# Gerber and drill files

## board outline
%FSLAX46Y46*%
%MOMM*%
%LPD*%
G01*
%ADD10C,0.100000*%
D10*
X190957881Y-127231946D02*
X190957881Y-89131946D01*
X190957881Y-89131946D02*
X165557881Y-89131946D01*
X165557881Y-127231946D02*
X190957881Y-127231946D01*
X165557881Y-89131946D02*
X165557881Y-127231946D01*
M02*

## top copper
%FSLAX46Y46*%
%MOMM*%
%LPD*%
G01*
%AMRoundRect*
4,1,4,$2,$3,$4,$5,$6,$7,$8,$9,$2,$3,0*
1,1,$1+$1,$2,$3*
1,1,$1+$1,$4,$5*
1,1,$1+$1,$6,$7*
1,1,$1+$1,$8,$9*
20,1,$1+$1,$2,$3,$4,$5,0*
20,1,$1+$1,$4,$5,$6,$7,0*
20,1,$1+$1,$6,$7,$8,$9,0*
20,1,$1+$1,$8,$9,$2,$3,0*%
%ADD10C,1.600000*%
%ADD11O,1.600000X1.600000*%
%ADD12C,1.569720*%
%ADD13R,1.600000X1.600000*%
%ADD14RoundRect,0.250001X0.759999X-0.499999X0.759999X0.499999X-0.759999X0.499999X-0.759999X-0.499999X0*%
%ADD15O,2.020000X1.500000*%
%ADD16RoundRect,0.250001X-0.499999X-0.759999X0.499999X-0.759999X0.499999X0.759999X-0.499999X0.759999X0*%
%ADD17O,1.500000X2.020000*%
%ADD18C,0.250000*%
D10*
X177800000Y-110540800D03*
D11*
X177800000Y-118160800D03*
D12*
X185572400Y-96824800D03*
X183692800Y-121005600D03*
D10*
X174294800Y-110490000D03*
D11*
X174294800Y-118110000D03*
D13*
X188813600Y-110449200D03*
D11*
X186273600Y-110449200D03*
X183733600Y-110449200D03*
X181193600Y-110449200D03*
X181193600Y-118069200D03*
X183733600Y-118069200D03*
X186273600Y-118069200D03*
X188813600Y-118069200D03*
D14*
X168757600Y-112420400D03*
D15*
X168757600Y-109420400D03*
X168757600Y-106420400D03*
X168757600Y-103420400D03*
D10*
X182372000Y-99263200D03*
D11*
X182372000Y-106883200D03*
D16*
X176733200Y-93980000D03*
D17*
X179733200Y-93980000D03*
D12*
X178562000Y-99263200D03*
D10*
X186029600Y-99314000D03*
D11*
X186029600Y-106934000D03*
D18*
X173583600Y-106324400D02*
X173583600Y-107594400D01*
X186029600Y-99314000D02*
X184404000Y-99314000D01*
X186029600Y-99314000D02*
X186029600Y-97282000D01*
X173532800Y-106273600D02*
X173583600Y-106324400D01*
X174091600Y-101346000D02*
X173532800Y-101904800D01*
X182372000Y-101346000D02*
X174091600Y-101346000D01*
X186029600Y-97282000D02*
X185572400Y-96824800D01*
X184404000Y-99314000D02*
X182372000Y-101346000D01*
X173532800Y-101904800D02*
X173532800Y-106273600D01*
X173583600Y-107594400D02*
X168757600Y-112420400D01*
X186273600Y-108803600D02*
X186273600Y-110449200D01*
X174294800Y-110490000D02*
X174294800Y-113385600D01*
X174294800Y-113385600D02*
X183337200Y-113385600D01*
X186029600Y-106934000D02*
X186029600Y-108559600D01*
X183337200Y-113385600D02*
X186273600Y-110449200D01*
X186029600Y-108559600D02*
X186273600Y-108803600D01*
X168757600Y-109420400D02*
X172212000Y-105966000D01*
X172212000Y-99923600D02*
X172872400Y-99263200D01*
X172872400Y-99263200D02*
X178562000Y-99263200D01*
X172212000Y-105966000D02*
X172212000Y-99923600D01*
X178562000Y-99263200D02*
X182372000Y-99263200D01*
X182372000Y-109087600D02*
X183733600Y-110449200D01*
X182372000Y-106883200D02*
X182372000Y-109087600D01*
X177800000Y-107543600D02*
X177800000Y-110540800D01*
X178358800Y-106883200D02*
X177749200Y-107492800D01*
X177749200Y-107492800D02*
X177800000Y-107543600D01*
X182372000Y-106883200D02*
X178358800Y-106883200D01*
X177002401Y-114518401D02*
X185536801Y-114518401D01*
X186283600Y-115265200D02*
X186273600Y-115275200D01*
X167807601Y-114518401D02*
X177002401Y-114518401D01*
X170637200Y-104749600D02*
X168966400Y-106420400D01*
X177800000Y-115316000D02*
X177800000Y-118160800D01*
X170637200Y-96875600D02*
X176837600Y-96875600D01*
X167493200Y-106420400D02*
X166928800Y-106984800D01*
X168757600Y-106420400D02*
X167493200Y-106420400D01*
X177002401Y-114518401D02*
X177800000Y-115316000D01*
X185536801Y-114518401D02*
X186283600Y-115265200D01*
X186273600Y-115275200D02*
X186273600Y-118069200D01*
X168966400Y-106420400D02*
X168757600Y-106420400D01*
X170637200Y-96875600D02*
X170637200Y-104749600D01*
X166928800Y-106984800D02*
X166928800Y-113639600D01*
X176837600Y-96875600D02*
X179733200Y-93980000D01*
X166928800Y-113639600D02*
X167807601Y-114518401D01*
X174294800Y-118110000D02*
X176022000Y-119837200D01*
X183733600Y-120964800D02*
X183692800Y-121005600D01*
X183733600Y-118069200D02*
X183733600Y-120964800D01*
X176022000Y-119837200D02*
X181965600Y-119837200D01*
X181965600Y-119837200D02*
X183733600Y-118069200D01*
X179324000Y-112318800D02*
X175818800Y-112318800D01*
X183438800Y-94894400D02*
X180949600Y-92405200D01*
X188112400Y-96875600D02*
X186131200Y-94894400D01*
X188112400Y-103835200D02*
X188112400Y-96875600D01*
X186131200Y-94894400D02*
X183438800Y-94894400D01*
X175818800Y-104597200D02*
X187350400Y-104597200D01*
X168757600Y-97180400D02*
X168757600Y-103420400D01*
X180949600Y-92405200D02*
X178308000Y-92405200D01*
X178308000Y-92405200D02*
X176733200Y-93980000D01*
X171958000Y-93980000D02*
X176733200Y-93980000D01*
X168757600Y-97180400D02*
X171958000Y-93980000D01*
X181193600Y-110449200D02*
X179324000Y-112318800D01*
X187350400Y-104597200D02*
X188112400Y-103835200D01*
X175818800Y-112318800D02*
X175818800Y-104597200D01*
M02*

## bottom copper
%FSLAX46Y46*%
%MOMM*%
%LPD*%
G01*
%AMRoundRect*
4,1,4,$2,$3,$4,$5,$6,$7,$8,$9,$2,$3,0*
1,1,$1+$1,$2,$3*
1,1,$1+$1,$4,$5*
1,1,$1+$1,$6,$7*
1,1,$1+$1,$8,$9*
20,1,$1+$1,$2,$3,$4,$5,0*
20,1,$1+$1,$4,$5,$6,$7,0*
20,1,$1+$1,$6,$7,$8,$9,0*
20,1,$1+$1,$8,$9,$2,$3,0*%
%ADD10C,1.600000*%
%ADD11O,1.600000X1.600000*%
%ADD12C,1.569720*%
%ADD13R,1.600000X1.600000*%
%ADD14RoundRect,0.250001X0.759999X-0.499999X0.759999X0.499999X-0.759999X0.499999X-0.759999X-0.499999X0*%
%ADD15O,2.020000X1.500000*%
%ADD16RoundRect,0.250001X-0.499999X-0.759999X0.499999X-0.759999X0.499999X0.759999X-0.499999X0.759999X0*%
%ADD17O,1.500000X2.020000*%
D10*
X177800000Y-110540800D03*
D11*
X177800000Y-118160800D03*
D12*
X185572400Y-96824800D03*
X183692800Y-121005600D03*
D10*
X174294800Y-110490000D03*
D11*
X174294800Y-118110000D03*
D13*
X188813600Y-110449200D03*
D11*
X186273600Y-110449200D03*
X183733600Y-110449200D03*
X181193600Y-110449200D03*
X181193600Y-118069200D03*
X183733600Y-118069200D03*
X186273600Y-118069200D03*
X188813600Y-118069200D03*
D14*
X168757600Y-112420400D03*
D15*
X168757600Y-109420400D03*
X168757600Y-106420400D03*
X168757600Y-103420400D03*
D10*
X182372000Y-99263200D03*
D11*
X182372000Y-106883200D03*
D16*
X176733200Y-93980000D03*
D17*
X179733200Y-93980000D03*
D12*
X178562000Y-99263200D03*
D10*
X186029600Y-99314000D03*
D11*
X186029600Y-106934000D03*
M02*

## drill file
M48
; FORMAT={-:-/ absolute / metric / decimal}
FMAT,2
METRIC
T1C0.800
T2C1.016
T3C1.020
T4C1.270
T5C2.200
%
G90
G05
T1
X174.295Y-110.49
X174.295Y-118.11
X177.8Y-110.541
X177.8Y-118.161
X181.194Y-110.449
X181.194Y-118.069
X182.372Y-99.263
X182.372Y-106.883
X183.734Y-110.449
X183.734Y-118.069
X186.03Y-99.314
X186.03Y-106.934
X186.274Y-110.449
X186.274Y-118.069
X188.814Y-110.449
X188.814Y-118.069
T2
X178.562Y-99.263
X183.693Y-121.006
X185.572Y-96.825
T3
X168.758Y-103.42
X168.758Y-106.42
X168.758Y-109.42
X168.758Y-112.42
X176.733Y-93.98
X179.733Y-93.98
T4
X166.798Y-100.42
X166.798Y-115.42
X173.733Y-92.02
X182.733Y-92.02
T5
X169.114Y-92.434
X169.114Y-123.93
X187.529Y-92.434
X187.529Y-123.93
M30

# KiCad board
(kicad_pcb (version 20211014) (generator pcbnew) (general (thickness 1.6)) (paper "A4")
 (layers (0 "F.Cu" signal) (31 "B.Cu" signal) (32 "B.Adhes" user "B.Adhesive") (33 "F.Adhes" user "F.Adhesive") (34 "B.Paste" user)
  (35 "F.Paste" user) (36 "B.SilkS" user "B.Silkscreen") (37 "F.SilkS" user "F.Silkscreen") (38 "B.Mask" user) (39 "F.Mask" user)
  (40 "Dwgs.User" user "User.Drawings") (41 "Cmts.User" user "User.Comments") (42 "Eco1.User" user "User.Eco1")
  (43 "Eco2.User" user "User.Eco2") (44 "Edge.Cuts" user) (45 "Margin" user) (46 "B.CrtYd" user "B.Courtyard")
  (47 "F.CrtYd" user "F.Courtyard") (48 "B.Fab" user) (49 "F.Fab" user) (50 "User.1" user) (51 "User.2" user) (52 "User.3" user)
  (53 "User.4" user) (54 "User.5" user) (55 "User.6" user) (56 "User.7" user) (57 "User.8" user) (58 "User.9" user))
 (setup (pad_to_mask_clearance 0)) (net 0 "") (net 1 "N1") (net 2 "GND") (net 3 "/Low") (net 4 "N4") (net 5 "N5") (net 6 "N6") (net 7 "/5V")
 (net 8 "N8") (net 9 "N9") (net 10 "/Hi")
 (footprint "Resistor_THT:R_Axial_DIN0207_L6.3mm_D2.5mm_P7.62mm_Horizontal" (layer "F.Cu") (at 177.8 110.5408 -90)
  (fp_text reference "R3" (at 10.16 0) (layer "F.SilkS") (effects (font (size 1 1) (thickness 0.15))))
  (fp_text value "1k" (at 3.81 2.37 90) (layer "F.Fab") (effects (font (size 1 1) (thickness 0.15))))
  (pad "1" thru_hole circle (at 0 0 270) (size 1.6 1.6) (drill 0.8) (layers *.Cu *.Mask) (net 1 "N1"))
  (pad "2" thru_hole oval (at 7.62 0 270) (size 1.6 1.6) (drill 0.8) (layers *.Cu *.Mask) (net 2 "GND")))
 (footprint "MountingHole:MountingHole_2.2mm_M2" (layer "F.Cu") (at 187.528881 123.929946)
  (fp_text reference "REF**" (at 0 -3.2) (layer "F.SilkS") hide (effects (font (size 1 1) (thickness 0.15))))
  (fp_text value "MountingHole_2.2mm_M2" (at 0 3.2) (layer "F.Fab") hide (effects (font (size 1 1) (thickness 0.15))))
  (pad "" np_thru_hole circle (at 0 0) (size 2.2 2.2) (drill 2.2) (layers F&B.Cu *.Mask)))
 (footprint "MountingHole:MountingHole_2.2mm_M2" (layer "F.Cu") (at 169.113881 92.433946)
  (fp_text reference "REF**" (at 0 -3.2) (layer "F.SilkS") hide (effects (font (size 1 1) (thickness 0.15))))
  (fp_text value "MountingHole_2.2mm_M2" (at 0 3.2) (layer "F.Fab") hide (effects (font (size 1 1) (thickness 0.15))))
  (pad "" np_thru_hole circle (at 0 0) (size 2.2 2.2) (drill 2.2) (layers F&B.Cu *.Mask)))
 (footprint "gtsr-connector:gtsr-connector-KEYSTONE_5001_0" (layer "F.Cu") (at 185.5724 96.8248)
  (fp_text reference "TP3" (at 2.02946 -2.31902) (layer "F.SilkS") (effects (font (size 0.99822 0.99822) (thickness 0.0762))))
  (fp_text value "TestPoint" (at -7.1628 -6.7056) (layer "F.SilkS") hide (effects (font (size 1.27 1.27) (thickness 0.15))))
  (pad "1" thru_hole circle (at 0 0) (size 1.56972 1.56972) (drill 1.016) (layers *.Cu *.Paste *.Mask) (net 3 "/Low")))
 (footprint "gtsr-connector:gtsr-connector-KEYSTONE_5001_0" (layer "F.Cu") (at 183.6928 121.0056)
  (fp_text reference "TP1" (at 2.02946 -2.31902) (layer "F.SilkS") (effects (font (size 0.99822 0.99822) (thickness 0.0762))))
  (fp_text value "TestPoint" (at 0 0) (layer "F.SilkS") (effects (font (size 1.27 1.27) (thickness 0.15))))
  (pad "1" thru_hole circle (at 0 0) (size 1.56972 1.56972) (drill 1.016) (layers *.Cu *.Paste *.Mask) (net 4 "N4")))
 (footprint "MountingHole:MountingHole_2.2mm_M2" (layer "F.Cu") (at 169.113881 123.929946)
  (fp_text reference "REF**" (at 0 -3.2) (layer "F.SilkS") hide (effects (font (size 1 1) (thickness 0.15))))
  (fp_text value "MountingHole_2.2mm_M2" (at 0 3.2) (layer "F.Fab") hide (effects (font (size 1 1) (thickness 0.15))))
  (pad "" np_thru_hole circle (at 0 0) (size 2.2 2.2) (drill 2.2) (layers F&B.Cu *.Mask)))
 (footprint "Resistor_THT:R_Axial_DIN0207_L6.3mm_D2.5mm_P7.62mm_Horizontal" (layer "F.Cu") (at 174.2948 110.49 -90)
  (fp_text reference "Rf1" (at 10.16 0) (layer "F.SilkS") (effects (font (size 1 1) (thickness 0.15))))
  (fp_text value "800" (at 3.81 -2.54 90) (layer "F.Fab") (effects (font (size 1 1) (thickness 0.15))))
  (pad "1" thru_hole circle (at 0 0 270) (size 1.6 1.6) (drill 0.8) (layers *.Cu *.Mask) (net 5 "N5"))
  (pad "2" thru_hole oval (at 7.62 0 270) (size 1.6 1.6) (drill 0.8) (layers *.Cu *.Mask) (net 4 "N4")))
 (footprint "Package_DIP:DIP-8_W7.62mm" (layer "F.Cu") (at 188.8136 110.4492 -90)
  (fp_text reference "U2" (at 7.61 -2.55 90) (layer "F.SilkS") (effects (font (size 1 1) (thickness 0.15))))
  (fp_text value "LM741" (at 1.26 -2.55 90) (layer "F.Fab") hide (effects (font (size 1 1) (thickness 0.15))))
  (pad "1" thru_hole rect (at 0 0 270) (size 1.6 1.6) (drill 0.8) (layers *.Cu *.Mask) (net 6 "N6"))
  (pad "2" thru_hole oval (at 0 2.54 270) (size 1.6 1.6) (drill 0.8) (layers *.Cu *.Mask) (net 5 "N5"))
  (pad "3" thru_hole oval (at 0 5.08 270) (size 1.6 1.6) (drill 0.8) (layers *.Cu *.Mask) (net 1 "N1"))
  (pad "4" thru_hole oval (at 0 7.62 270) (size 1.6 1.6) (drill 0.8) (layers *.Cu *.Mask) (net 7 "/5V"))
  (pad "5" thru_hole oval (at 7.62 7.62 270) (size 1.6 1.6) (drill 0.8) (layers *.Cu *.Mask) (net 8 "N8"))
  (pad "6" thru_hole oval (at 7.62 5.08 270) (size 1.6 1.6) (drill 0.8) (layers *.Cu *.Mask) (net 4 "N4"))
  (pad "7" thru_hole oval (at 7.62 2.54 270) (size 1.6 1.6) (drill 0.8) (layers *.Cu *.Mask) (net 2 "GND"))
  (pad "8" thru_hole oval (at 7.62 0 270) (size 1.6 1.6) (drill 0.8) (layers *.Cu *.Mask) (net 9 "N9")))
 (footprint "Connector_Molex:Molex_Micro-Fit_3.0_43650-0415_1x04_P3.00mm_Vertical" (layer "F.Cu") (at 168.7576 112.4204 90)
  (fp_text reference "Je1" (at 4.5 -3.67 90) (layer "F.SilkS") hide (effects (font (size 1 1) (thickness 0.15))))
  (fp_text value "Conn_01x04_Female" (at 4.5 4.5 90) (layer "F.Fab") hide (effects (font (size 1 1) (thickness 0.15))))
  (pad "" np_thru_hole circle (at -3 -1.96 90) (size 1.27 1.27) (drill 1.27) (layers *.Cu *.Mask))
  (pad "" np_thru_hole circle (at 12 -1.96 90) (size 1.27 1.27) (drill 1.27) (layers *.Cu *.Mask))
  (pad "1" thru_hole roundrect (at 0 0 90) (size 1.5 2.02) (drill 1.02) (layers *.Cu *.Mask) (roundrect_rratio 0.166667) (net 3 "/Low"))
  (pad "2" thru_hole oval (at 3 0 90) (size 1.5 2.02) (drill 1.02) (layers *.Cu *.Mask) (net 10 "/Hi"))
  (pad "3" thru_hole oval (at 6 0 90) (size 1.5 2.02) (drill 1.02) (layers *.Cu *.Mask) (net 2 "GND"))
  (pad "4" thru_hole oval (at 9 0 90) (size 1.5 2.02) (drill 1.02) (layers *.Cu *.Mask) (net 7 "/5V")))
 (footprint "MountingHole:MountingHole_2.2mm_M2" (layer "F.Cu") (at 187.528881 92.433946)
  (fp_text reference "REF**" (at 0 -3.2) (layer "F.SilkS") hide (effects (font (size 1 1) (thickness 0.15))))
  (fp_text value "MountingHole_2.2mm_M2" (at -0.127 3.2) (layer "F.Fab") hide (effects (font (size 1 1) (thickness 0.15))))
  (pad "" np_thru_hole circle (at 0 0) (size 2.2 2.2) (drill 2.2) (layers *.Cu *.Mask)))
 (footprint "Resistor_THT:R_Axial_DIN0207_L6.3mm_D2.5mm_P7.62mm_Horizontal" (layer "F.Cu") (at 182.372 99.2632 -90)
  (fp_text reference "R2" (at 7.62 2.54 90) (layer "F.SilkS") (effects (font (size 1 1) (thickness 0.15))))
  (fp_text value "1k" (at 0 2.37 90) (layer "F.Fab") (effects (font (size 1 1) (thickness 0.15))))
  (pad "1" thru_hole circle (at 0 0 270) (size 1.6 1.6) (drill 0.8) (layers *.Cu *.Mask) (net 10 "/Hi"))
  (pad "2" thru_hole oval (at 7.62 0 270) (size 1.6 1.6) (drill 0.8) (layers *.Cu *.Mask) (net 1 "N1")))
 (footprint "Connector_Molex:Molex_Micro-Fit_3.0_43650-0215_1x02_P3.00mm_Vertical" (layer "F.Cu") (at 176.7332 93.98)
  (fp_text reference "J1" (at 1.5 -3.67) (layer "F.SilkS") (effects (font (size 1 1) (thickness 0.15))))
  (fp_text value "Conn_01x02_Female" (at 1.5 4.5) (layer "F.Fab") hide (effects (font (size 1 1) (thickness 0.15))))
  (pad "" np_thru_hole circle (at 6 -1.96) (size 1.27 1.27) (drill 1.27) (layers *.Cu *.Mask))
  (pad "" np_thru_hole circle (at -3 -1.96) (size 1.27 1.27) (drill 1.27) (layers *.Cu *.Mask))
  (pad "1" thru_hole roundrect (at 0 0) (size 1.5 2.02) (drill 1.02) (layers *.Cu *.Mask) (roundrect_rratio 0.166667) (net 7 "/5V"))
  (pad "2" thru_hole oval (at 3 0) (size 1.5 2.02) (drill 1.02) (layers *.Cu *.Mask) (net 2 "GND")))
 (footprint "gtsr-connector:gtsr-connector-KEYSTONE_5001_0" (layer "F.Cu") (at 178.562 99.2632)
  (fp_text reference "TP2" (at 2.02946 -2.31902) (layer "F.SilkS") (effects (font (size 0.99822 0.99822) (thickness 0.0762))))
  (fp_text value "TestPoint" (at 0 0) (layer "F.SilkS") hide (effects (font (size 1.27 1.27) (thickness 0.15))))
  (pad "1" thru_hole circle (at 0 0) (size 1.56972 1.56972) (drill 1.016) (layers *.Cu *.Paste *.Mask) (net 10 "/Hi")))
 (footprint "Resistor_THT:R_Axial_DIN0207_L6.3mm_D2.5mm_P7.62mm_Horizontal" (layer "F.Cu") (at 186.0296 99.314 -90)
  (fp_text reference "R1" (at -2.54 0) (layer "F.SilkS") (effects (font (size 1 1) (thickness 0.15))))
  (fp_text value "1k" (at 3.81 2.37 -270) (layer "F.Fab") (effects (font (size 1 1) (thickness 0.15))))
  (pad "1" thru_hole circle (at 0 0 270) (size 1.6 1.6) (drill 0.8) (layers *.Cu *.Mask) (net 3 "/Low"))
  (pad "2" thru_hole oval (at 7.62 0 270) (size 1.6 1.6) (drill 0.8) (layers *.Cu *.Mask) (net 5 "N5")))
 (gr_line (start 190.957881 127.231946) (end 190.957881 89.131946) (layer "Edge.Cuts") (width 0.1))
 (gr_line (start 190.957881 89.131946) (end 165.557881 89.131946) (layer "Edge.Cuts") (width 0.1))
 (gr_line (start 165.557881 127.231946) (end 190.957881 127.231946) (layer "Edge.Cuts") (width 0.1))
 (gr_line (start 165.557881 89.131946) (end 165.557881 127.231946) (layer "Edge.Cuts") (width 0.1))
 (segment (start 173.5836 106.3244) (end 173.5836 107.5944) (width 0.25) (layer "F.Cu") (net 3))
 (segment (start 186.0296 99.314) (end 184.404 99.314) (width 0.25) (layer "F.Cu") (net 3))
 (segment (start 186.0296 99.314) (end 186.0296 97.282) (width 0.25) (layer "F.Cu") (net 3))
 (segment (start 173.5328 106.2736) (end 173.5836 106.3244) (width 0.25) (layer "F.Cu") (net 3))
 (segment (start 174.0916 101.346) (end 173.5328 101.9048) (width 0.25) (layer "F.Cu") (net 3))
 (segment (start 182.372 101.346) (end 174.0916 101.346) (width 0.25) (layer "F.Cu") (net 3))
 (segment (start 186.0296 97.282) (end 185.5724 96.8248) (width 0.25) (layer "F.Cu") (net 3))
 (segment (start 184.404 99.314) (end 182.372 101.346) (width 0.25) (layer "F.Cu") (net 3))
 (segment (start 173.5328 101.9048) (end 173.5328 106.2736) (width 0.25) (layer "F.Cu") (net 3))
 (segment (start 173.5836 107.5944) (end 168.7576 112.4204) (width 0.25) (layer "F.Cu") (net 3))
 (segment (start 186.2736 108.8036) (end 186.2736 110.4492) (width 0.25) (layer "F.Cu") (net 5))
 (segment (start 174.2948 110.49) (end 174.2948 113.3856) (width 0.25) (layer "F.Cu") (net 5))
 (segment (start 174.2948 113.3856) (end 183.3372 113.3856) (width 0.25) (layer "F.Cu") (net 5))
 (segment (start 186.0296 106.934) (end 186.0296 108.5596) (width 0.25) (layer "F.Cu") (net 5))
 (segment (start 183.3372 113.3856) (end 186.2736 110.4492) (width 0.25) (layer "F.Cu") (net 5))
 (segment (start 186.0296 108.5596) (end 186.2736 108.8036) (width 0.25) (layer "F.Cu") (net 5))
 (segment (start 168.7576 109.4204) (end 172.212 105.966) (width 0.25) (layer "F.Cu") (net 10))
 (segment (start 172.212 99.9236) (end 172.8724 99.2632) (width 0.25) (layer "F.Cu") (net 10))
 (segment (start 172.8724 99.2632) (end 178.562 99.2632) (width 0.25) (layer "F.Cu") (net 10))
 (segment (start 172.212 105.966) (end 172.212 99.9236) (width 0.25) (layer "F.Cu") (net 10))
 (segment (start 178.562 99.2632) (end 182.372 99.2632) (width 0.25) (layer "F.Cu") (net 10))
 (segment (start 182.372 109.0876) (end 183.7336 110.4492) (width 0.25) (layer "F.Cu") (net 1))
 (segment (start 182.372 106.8832) (end 182.372 109.0876) (width 0.25) (layer "F.Cu") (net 1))
 (segment (start 177.8 107.5436) (end 177.8 110.5408) (width 0.25) (layer "F.Cu") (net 1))
 (segment (start 178.3588 106.8832) (end 177.7492 107.4928) (width 0.25) (layer "F.Cu") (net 1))
 (segment (start 177.7492 107.4928) (end 177.8 107.5436) (width 0.25) (layer "F.Cu") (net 1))
 (segment (start 182.372 106.8832) (end 178.3588 106.8832) (width 0.25) (layer "F.Cu") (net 1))
 (segment (start 177.002401 114.518401) (end 185.536801 114.518401) (width 0.25) (layer "F.Cu") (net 2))
 (segment (start 186.2836 115.2652) (end 186.2736 115.2752) (width 0.25) (layer "F.Cu") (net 2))
 (segment (start 167.807601 114.518401) (end 177.002401 114.518401) (width 0.25) (layer "F.Cu") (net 2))
 (segment (start 170.6372 104.7496) (end 168.9664 106.4204) (width 0.25) (layer "F.Cu") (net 2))
 (segment (start 177.8 115.316) (end 177.8 118.1608) (width 0.25) (layer "F.Cu") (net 2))
 (segment (start 170.6372 96.8756) (end 176.8376 96.8756) (width 0.25) (layer "F.Cu") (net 2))
 (segment (start 167.4932 106.4204) (end 166.9288 106.9848) (width 0.25) (layer "F.Cu") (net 2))
 (segment (start 168.7576 106.4204) (end 167.4932 106.4204) (width 0.25) (layer "F.Cu") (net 2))
 (segment (start 177.002401 114.518401) (end 177.8 115.316) (width 0.25) (layer "F.Cu") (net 2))
 (segment (start 185.536801 114.518401) (end 186.2836 115.2652) (width 0.25) (layer "F.Cu") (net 2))
 (segment (start 186.2736 115.2752) (end 186.2736 118.0692) (width 0.25) (layer "F.Cu") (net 2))
 (segment (start 168.9664 106.4204) (end 168.7576 106.4204) (width 0.25) (layer "F.Cu") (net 2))
 (segment (start 170.6372 96.8756) (end 170.6372 104.7496) (width 0.25) (layer "F.Cu") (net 2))
 (segment (start 166.9288 106.9848) (end 166.9288 113.6396) (width 0.25) (layer "F.Cu") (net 2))
 (segment (start 176.8376 96.8756) (end 179.7332 93.98) (width 0.25) (layer "F.Cu") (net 2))
 (segment (start 166.9288 113.6396) (end 167.807601 114.518401) (width 0.25) (layer "F.Cu") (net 2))
 (segment (start 174.2948 118.11) (end 176.022 119.8372) (width 0.25) (layer "F.Cu") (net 4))
 (segment (start 183.7336 120.9648) (end 183.6928 121.0056) (width 0.25) (layer "F.Cu") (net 4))
 (segment (start 183.7336 118.0692) (end 183.7336 120.9648) (width 0.25) (layer "F.Cu") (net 4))
 (segment (start 176.022 119.8372) (end 181.9656 119.8372) (width 0.25) (layer "F.Cu") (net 4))
 (segment (start 181.9656 119.8372) (end 183.7336 118.0692) (width 0.25) (layer "F.Cu") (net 4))
 (segment (start 179.324 112.3188) (end 175.8188 112.3188) (width 0.25) (layer "F.Cu") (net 7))
 (segment (start 183.4388 94.8944) (end 180.9496 92.4052) (width 0.25) (layer "F.Cu") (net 7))
 (segment (start 188.1124 96.8756) (end 186.1312 94.8944) (width 0.25) (layer "F.Cu") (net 7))
 (segment (start 188.1124 103.8352) (end 188.1124 96.8756) (width 0.25) (layer "F.Cu") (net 7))
 (segment (start 186.1312 94.8944) (end 183.4388 94.8944) (width 0.25) (layer "F.Cu") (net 7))
 (segment (start 175.8188 104.5972) (end 187.3504 104.5972) (width 0.25) (layer "F.Cu") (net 7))
 (segment (start 168.7576 97.1804) (end 168.7576 103.4204) (width 0.25) (layer "F.Cu") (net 7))
 (segment (start 180.9496 92.4052) (end 178.308 92.4052) (width 0.25) (layer "F.Cu") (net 7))
 (segment (start 178.308 92.4052) (end 176.7332 93.98) (width 0.25) (layer "F.Cu") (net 7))
 (segment (start 171.958 93.98) (end 176.7332 93.98) (width 0.25) (layer "F.Cu") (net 7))
 (segment (start 168.7576 97.1804) (end 171.958 93.98) (width 0.25) (layer "F.Cu") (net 7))
 (segment (start 181.1936 110.4492) (end 179.324 112.3188) (width 0.25) (layer "F.Cu") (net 7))
 (segment (start 187.3504 104.5972) (end 188.1124 103.8352) (width 0.25) (layer "F.Cu") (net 7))
 (segment (start 175.8188 112.3188) (end 175.8188 104.5972) (width 0.25) (layer "F.Cu") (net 7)))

